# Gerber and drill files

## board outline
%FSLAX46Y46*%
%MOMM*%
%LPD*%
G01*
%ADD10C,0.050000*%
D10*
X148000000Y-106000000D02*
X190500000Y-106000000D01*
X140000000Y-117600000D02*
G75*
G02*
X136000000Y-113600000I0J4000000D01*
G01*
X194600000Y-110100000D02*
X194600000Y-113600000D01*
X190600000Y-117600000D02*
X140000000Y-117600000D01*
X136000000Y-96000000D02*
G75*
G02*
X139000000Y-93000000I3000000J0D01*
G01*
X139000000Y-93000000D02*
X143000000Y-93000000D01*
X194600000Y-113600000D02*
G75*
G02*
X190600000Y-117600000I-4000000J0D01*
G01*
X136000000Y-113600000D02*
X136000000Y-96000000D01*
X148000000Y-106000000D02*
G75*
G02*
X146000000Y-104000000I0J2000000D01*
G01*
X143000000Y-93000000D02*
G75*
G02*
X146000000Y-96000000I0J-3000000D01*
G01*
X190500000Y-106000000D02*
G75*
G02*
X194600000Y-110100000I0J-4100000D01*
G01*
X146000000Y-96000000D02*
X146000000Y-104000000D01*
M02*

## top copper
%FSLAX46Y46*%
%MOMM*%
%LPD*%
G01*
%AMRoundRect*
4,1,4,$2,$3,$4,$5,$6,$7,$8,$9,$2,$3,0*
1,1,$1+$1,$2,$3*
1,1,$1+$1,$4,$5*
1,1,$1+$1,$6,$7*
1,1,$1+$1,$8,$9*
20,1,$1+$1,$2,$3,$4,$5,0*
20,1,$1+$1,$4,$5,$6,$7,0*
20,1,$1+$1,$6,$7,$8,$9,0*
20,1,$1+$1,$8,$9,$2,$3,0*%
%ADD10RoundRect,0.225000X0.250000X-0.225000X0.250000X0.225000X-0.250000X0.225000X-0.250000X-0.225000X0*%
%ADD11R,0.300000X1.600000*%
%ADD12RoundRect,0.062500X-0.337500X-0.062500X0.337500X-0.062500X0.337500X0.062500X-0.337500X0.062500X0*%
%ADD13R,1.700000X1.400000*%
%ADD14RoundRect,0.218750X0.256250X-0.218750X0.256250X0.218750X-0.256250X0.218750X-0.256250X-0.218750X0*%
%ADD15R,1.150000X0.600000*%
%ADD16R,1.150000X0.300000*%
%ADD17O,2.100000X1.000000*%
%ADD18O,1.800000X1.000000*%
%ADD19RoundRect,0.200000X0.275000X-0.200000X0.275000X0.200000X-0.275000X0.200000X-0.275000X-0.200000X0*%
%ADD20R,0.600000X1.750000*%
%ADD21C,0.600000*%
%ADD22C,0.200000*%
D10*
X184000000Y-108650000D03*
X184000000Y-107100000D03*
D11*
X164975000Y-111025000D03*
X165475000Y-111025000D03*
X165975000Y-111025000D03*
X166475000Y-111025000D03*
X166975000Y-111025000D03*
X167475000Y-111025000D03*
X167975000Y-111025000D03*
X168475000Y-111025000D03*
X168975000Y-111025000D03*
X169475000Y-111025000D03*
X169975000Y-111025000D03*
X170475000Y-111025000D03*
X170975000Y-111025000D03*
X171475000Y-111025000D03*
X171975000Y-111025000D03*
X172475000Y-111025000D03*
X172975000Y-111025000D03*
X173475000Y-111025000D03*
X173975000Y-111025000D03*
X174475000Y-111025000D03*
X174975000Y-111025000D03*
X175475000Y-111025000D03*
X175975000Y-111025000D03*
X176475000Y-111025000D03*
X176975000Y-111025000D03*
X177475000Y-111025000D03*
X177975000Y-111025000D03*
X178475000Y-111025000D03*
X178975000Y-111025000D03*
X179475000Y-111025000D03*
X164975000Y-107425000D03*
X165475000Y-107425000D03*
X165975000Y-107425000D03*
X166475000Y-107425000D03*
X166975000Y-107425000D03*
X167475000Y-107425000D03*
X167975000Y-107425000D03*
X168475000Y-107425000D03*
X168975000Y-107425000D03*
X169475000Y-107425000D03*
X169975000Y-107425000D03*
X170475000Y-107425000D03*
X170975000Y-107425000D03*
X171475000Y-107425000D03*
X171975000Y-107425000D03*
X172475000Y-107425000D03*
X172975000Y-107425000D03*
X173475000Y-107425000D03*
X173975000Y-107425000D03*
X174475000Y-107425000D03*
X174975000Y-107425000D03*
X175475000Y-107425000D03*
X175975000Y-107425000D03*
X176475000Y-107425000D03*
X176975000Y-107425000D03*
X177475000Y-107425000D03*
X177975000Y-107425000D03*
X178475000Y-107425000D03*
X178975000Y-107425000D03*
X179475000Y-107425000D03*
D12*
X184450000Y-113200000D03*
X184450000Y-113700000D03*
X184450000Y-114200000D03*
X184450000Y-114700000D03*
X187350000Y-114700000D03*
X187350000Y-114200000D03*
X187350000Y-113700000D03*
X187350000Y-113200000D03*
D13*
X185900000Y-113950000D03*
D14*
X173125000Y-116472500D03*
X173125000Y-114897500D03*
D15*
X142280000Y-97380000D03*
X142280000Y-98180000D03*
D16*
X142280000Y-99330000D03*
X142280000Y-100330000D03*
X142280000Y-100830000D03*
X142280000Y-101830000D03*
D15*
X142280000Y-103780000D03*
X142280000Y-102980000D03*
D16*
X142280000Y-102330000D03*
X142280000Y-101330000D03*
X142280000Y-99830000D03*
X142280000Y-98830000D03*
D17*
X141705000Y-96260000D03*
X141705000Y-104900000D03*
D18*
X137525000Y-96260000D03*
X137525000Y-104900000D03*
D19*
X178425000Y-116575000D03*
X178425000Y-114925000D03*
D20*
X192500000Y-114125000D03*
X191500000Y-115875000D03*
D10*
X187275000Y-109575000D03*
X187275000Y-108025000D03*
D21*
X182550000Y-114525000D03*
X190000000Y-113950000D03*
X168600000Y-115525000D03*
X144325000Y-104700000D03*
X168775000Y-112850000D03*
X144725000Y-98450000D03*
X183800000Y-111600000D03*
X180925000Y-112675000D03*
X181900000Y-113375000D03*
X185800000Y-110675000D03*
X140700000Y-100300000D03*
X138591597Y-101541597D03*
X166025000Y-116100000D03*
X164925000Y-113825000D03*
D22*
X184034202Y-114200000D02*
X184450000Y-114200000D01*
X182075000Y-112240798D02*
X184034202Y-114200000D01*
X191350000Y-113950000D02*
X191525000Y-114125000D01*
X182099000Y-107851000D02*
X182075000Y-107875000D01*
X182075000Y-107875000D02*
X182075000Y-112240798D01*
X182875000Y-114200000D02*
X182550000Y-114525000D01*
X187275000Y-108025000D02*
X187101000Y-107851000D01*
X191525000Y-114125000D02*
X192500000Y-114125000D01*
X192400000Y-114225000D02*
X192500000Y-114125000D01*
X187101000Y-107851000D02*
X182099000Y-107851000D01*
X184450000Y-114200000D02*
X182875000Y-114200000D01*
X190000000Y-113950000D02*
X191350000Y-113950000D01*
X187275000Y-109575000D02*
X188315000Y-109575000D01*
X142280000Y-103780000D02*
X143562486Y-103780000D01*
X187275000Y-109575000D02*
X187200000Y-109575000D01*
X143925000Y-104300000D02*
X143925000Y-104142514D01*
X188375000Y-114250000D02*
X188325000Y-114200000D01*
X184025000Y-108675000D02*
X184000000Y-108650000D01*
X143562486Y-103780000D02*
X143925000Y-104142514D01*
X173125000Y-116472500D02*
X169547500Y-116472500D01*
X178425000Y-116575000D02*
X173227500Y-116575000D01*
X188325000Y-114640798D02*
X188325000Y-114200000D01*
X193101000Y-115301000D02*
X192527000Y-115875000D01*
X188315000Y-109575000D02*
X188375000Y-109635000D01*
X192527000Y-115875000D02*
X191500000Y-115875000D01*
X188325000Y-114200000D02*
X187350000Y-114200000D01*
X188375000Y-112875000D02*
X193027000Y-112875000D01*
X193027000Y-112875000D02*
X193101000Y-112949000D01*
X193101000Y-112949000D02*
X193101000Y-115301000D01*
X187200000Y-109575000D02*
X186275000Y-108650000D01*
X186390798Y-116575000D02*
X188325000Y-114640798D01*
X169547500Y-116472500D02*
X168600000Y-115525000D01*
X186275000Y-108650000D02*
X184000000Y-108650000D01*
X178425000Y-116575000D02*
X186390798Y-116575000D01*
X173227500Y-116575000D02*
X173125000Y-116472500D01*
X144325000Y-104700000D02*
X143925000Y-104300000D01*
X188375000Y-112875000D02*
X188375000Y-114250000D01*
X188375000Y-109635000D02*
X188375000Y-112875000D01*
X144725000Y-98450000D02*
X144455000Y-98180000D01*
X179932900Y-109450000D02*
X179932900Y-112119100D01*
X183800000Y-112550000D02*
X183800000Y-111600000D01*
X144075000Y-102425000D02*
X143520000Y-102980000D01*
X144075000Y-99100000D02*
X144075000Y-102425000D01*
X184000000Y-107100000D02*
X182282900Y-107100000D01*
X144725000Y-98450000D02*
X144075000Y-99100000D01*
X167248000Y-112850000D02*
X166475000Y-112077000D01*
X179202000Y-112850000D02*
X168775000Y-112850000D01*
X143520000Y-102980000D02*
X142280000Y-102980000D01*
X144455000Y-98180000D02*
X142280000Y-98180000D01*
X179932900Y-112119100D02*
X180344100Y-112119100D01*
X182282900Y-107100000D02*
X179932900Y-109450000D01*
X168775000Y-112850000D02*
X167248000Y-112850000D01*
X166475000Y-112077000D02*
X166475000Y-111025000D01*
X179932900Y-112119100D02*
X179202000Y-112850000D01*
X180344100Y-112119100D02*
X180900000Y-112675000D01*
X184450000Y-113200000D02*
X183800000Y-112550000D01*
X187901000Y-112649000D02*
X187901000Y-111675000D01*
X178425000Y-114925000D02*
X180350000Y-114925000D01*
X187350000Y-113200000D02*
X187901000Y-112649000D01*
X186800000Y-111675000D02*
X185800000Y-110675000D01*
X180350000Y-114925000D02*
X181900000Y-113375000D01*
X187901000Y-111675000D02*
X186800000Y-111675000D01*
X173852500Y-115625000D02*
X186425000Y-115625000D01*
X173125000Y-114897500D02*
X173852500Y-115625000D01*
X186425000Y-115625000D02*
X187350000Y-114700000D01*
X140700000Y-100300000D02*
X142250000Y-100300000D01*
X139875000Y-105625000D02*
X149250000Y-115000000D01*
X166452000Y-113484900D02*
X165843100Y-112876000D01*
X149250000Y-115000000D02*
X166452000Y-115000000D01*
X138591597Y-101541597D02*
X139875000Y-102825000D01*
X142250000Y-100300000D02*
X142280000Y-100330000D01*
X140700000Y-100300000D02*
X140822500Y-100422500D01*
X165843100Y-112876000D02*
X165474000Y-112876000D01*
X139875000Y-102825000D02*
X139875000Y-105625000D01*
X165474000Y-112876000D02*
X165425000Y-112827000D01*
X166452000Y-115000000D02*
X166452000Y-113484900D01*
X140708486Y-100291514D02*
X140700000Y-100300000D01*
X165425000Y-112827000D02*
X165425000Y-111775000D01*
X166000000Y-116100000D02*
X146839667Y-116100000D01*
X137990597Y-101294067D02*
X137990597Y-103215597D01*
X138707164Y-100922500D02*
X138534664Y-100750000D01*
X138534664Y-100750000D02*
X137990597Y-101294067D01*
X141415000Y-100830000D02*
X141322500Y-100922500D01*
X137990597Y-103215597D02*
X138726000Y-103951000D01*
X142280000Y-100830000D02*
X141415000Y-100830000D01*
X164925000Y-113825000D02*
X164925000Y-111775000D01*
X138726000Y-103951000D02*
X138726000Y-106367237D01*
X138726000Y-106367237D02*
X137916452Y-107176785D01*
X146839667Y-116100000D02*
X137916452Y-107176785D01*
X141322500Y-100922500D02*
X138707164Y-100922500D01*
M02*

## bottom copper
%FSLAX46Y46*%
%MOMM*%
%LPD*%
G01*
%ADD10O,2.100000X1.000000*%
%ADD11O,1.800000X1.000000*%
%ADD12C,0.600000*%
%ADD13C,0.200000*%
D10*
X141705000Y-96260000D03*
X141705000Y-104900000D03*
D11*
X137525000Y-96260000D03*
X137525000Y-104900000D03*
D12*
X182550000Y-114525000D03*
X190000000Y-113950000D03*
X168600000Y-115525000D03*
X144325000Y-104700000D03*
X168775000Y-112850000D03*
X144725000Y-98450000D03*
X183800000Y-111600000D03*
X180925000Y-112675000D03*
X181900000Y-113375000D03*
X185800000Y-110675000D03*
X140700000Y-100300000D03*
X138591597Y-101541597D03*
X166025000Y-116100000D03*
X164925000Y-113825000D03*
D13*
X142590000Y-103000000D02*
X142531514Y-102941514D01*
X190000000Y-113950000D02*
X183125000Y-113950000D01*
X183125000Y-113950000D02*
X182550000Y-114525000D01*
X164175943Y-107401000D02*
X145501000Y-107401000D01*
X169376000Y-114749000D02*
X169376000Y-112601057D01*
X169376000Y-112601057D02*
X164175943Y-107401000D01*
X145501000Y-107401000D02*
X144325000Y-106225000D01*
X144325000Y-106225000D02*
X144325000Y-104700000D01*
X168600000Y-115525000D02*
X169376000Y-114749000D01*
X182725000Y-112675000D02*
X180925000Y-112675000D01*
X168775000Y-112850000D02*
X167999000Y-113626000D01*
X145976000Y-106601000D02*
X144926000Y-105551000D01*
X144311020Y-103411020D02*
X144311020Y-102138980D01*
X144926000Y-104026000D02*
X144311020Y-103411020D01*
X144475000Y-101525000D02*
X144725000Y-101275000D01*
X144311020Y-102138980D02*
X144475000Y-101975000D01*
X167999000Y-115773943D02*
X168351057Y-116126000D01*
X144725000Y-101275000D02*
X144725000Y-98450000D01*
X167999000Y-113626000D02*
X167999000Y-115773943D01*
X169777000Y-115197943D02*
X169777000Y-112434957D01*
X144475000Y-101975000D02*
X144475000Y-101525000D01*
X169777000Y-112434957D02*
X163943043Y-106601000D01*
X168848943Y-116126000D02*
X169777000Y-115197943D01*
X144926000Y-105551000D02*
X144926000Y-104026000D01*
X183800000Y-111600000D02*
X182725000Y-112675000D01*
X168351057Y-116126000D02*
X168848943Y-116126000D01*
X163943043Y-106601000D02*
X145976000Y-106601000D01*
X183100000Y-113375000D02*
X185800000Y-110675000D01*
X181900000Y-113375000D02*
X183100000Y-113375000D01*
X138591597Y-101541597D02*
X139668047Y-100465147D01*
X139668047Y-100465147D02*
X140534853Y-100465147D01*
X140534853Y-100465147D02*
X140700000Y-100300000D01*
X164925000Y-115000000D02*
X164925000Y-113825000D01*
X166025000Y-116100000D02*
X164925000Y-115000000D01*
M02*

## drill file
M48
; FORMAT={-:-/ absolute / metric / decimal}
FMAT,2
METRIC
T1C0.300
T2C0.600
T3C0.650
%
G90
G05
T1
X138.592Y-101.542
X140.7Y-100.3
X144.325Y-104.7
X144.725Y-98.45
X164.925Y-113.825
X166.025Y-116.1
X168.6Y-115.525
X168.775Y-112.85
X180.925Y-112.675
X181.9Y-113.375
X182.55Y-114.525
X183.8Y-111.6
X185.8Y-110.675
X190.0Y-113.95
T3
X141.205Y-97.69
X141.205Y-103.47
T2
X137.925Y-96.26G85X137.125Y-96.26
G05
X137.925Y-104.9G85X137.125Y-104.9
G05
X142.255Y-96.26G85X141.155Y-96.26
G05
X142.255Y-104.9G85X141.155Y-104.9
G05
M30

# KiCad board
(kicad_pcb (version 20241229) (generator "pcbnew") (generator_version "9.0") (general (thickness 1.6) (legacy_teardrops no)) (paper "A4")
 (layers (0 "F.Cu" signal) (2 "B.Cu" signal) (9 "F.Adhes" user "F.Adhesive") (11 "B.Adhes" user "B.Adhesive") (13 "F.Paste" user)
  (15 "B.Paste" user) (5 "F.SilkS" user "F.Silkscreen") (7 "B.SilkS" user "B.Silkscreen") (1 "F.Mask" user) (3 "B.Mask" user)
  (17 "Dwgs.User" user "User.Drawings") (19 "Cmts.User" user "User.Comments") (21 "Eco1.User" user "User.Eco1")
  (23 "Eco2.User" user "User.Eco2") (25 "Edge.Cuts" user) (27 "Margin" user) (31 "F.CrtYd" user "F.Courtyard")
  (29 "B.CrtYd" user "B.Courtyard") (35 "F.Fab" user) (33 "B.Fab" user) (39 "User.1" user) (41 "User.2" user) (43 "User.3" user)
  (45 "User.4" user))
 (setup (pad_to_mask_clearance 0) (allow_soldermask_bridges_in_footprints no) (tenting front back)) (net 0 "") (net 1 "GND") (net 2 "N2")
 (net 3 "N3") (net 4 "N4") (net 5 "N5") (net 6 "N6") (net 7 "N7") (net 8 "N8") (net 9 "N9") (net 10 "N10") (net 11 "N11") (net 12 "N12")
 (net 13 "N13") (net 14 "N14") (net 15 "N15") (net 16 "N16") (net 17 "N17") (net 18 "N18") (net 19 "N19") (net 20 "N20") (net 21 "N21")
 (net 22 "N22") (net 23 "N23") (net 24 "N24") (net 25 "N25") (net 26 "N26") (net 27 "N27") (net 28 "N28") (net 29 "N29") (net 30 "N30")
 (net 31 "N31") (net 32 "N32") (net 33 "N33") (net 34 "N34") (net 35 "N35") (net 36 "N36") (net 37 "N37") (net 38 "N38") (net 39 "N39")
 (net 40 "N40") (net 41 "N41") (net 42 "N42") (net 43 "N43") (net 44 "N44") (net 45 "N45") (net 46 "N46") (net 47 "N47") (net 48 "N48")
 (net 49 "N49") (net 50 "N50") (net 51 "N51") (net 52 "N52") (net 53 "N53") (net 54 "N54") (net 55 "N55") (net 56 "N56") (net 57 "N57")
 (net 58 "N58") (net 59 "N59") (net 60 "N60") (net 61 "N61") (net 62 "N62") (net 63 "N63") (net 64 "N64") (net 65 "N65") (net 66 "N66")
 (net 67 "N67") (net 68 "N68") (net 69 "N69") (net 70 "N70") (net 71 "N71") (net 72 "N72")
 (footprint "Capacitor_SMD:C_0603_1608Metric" (layer "F.Cu") (at 184 107.875 90)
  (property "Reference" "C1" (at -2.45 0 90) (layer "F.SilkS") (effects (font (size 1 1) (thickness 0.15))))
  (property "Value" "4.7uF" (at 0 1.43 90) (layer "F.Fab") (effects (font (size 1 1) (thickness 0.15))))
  (pad "1" smd roundrect (at -0.775 0 90) (size 0.9 0.95) (layers "F.Cu" "F.Mask" "F.Paste") (roundrect_rratio 0.25) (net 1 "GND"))
  (pad "2" smd roundrect (at 0.775 0 90) (size 0.9 0.95) (layers "F.Cu" "F.Mask" "F.Paste") (roundrect_rratio 0.25) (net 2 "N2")))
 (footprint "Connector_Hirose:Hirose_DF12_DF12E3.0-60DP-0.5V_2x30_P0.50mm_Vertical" (layer "F.Cu") (at 172.225 109.225)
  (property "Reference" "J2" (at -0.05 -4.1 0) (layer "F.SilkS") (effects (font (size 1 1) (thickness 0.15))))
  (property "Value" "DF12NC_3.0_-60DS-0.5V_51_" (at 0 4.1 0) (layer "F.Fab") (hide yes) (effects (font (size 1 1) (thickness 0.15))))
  (pad "" smd rect (at -7.25 -2) (size 0.28 1.2) (layers "F.Paste"))
  (pad "" smd rect (at -7.25 2) (size 0.28 1.2) (layers "F.Paste"))
  (pad "" smd rect (at -6.75 -2) (size 0.28 1.2) (layers "F.Paste"))
  (pad "" smd rect (at -6.75 2) (size 0.28 1.2) (layers "F.Paste"))
  (pad "" smd rect (at -6.25 -2) (size 0.28 1.2) (layers "F.Paste"))
  (pad "" smd rect (at -6.25 2) (size 0.28 1.2) (layers "F.Paste"))
  (pad "" smd rect (at -5.75 -2) (size 0.28 1.2) (layers "F.Paste"))
  (pad "" smd rect (at -5.75 2) (size 0.28 1.2) (layers "F.Paste"))
  (pad "" smd rect (at -5.25 -2) (size 0.28 1.2) (layers "F.Paste"))
  (pad "" smd rect (at -5.25 2) (size 0.28 1.2) (layers "F.Paste"))
  (pad "" smd rect (at -4.75 -2) (size 0.28 1.2) (layers "F.Paste"))
  (pad "" smd rect (at -4.75 2) (size 0.28 1.2) (layers "F.Paste"))
  (pad "" smd rect (at -4.25 -2) (size 0.28 1.2) (layers "F.Paste"))
  (pad "" smd rect (at -4.25 2) (size 0.28 1.2) (layers "F.Paste"))
  (pad "" smd rect (at -3.75 -2) (size 0.28 1.2) (layers "F.Paste"))
  (pad "" smd rect (at -3.75 2) (size 0.28 1.2) (layers "F.Paste"))
  (pad "" smd rect (at -3.25 -2) (size 0.28 1.2) (layers "F.Paste"))
  (pad "" smd rect (at -3.25 2) (size 0.28 1.2) (layers "F.Paste"))
  (pad "" smd rect (at -2.75 -2) (size 0.28 1.2) (layers "F.Paste"))
  (pad "" smd rect (at -2.75 2) (size 0.28 1.2) (layers "F.Paste"))
  (pad "" smd rect (at -2.25 -2) (size 0.28 1.2) (layers "F.Paste"))
  (pad "" smd rect (at -2.25 2) (size 0.28 1.2) (layers "F.Paste"))
  (pad "" smd rect (at -1.75 -2) (size 0.28 1.2) (layers "F.Paste"))
  (pad "" smd rect (at -1.75 2) (size 0.28 1.2) (layers "F.Paste"))
  (pad "" smd rect (at -1.25 -2) (size 0.28 1.2) (layers "F.Paste"))
  (pad "" smd rect (at -1.25 2) (size 0.28 1.2) (layers "F.Paste"))
  (pad "" smd rect (at -0.75 -2) (size 0.28 1.2) (layers "F.Paste"))
  (pad "" smd rect (at -0.75 2) (size 0.28 1.2) (layers "F.Paste"))
  (pad "" smd rect (at -0.25 -2) (size 0.28 1.2) (layers "F.Paste"))
  (pad "" smd rect (at -0.25 2) (size 0.28 1.2) (layers "F.Paste"))
  (pad "" smd rect (at 0.25 -2) (size 0.28 1.2) (layers "F.Paste"))
  (pad "" smd rect (at 0.25 2) (size 0.28 1.2) (layers "F.Paste"))
  (pad "" smd rect (at 0.75 -2) (size 0.28 1.2) (layers "F.Paste"))
  (pad "" smd rect (at 0.75 2) (size 0.28 1.2) (layers "F.Paste"))
  (pad "" smd rect (at 1.25 -2) (size 0.28 1.2) (layers "F.Paste"))
  (pad "" smd rect (at 1.25 2) (size 0.28 1.2) (layers "F.Paste"))
  (pad "" smd rect (at 1.75 -2) (size 0.28 1.2) (layers "F.Paste"))
  (pad "" smd rect (at 1.75 2) (size 0.28 1.2) (layers "F.Paste"))
  (pad "" smd rect (at 2.25 -2) (size 0.28 1.2) (layers "F.Paste"))
  (pad "" smd rect (at 2.25 2) (size 0.28 1.2) (layers "F.Paste"))
  (pad "" smd rect (at 2.75 -2) (size 0.28 1.2) (layers "F.Paste"))
  (pad "" smd rect (at 2.75 2) (size 0.28 1.2) (layers "F.Paste"))
  (pad "" smd rect (at 3.25 -2) (size 0.28 1.2) (layers "F.Paste"))
  (pad "" smd rect (at 3.25 2) (size 0.28 1.2) (layers "F.Paste"))
  (pad "" smd rect (at 3.75 -2) (size 0.28 1.2) (layers "F.Paste"))
  (pad "" smd rect (at 3.75 2) (size 0.28 1.2) (layers "F.Paste"))
  (pad "" smd rect (at 4.25 -2) (size 0.28 1.2) (layers "F.Paste"))
  (pad "" smd rect (at 4.25 2) (size 0.28 1.2) (layers "F.Paste"))
  (pad "" smd rect (at 4.75 -2) (size 0.28 1.2) (layers "F.Paste"))
  (pad "" smd rect (at 4.75 2) (size 0.28 1.2) (layers "F.Paste"))
  (pad "" smd rect (at 5.25 -2) (size 0.28 1.2) (layers "F.Paste"))
  (pad "" smd rect (at 5.25 2) (size 0.28 1.2) (layers "F.Paste"))
  (pad "" smd rect (at 5.75 -2) (size 0.28 1.2) (layers "F.Paste"))
  (pad "" smd rect (at 5.75 2) (size 0.28 1.2) (layers "F.Paste"))
  (pad "" smd rect (at 6.25 -2) (size 0.28 1.2) (layers "F.Paste"))
  (pad "" smd rect (at 6.25 2) (size 0.28 1.2) (layers "F.Paste"))
  (pad "" smd rect (at 6.75 -2) (size 0.28 1.2) (layers "F.Paste"))
  (pad "" smd rect (at 6.75 2) (size 0.28 1.2) (layers "F.Paste"))
  (pad "" smd rect (at 7.25 -2) (size 0.28 1.2) (layers "F.Paste"))
  (pad "" smd rect (at 7.25 2) (size 0.28 1.2) (layers "F.Paste"))
  (pad "1" smd rect (at -7.25 1.8) (size 0.3 1.6) (layers "F.Cu" "F.Mask") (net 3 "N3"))
  (pad "2" smd rect (at -6.75 1.8) (size 0.3 1.6) (layers "F.Cu" "F.Mask") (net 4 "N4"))
  (pad "3" smd rect (at -6.25 1.8) (size 0.3 1.6) (layers "F.Cu" "F.Mask") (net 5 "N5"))
  (pad "4" smd rect (at -5.75 1.8) (size 0.3 1.6) (layers "F.Cu" "F.Mask") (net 2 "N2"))
  (pad "5" smd rect (at -5.25 1.8) (size 0.3 1.6) (layers "F.Cu" "F.Mask") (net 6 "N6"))
  (pad "6" smd rect (at -4.75 1.8) (size 0.3 1.6) (layers "F.Cu" "F.Mask") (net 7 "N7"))
  (pad "7" smd rect (at -4.25 1.8) (size 0.3 1.6) (layers "F.Cu" "F.Mask") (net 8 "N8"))
  (pad "8" smd rect (at -3.75 1.8) (size 0.3 1.6) (layers "F.Cu" "F.Mask") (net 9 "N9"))
  (pad "9" smd rect (at -3.25 1.8) (size 0.3 1.6) (layers "F.Cu" "F.Mask") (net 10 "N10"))
  (pad "10" smd rect (at -2.75 1.8) (size 0.3 1.6) (layers "F.Cu" "F.Mask") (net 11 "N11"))
  (pad "11" smd rect (at -2.25 1.8) (size 0.3 1.6) (layers "F.Cu" "F.Mask") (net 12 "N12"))
  (pad "12" smd rect (at -1.75 1.8) (size 0.3 1.6) (layers "F.Cu" "F.Mask") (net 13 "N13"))
  (pad "13" smd rect (at -1.25 1.8) (size 0.3 1.6) (layers "F.Cu" "F.Mask") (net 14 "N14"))
  (pad "14" smd rect (at -0.75 1.8) (size 0.3 1.6) (layers "F.Cu" "F.Mask") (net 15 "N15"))
  (pad "15" smd rect (at -0.25 1.8) (size 0.3 1.6) (layers "F.Cu" "F.Mask") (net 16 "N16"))
  (pad "16" smd rect (at 0.25 1.8) (size 0.3 1.6) (layers "F.Cu" "F.Mask") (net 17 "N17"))
  (pad "17" smd rect (at 0.75 1.8) (size 0.3 1.6) (layers "F.Cu" "F.Mask") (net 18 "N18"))
  (pad "18" smd rect (at 1.25 1.8) (size 0.3 1.6) (layers "F.Cu" "F.Mask") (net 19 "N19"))
  (pad "19" smd rect (at 1.75 1.8) (size 0.3 1.6) (layers "F.Cu" "F.Mask") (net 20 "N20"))
  (pad "20" smd rect (at 2.25 1.8) (size 0.3 1.6) (layers "F.Cu" "F.Mask") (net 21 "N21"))
  (pad "21" smd rect (at 2.75 1.8) (size 0.3 1.6) (layers "F.Cu" "F.Mask") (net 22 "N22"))
  (pad "22" smd rect (at 3.25 1.8) (size 0.3 1.6) (layers "F.Cu" "F.Mask") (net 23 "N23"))
  (pad "23" smd rect (at 3.75 1.8) (size 0.3 1.6) (layers "F.Cu" "F.Mask") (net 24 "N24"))
  (pad "24" smd rect (at 4.25 1.8) (size 0.3 1.6) (layers "F.Cu" "F.Mask") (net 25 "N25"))
  (pad "25" smd rect (at 4.75 1.8) (size 0.3 1.6) (layers "F.Cu" "F.Mask") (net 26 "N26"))
  (pad "26" smd rect (at 5.25 1.8) (size 0.3 1.6) (layers "F.Cu" "F.Mask") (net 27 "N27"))
  (pad "27" smd rect (at 5.75 1.8) (size 0.3 1.6) (layers "F.Cu" "F.Mask") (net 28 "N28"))
  (pad "28" smd rect (at 6.25 1.8) (size 0.3 1.6) (layers "F.Cu" "F.Mask") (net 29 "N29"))
  (pad "29" smd rect (at 6.75 1.8) (size 0.3 1.6) (layers "F.Cu" "F.Mask") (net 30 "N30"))
  (pad "30" smd rect (at 7.25 1.8) (size 0.3 1.6) (layers "F.Cu" "F.Mask") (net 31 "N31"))
  (pad "31" smd rect (at -7.25 -1.8) (size 0.3 1.6) (layers "F.Cu" "F.Mask") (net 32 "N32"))
  (pad "32" smd rect (at -6.75 -1.8) (size 0.3 1.6) (layers "F.Cu" "F.Mask") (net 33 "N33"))
  (pad "33" smd rect (at -6.25 -1.8) (size 0.3 1.6) (layers "F.Cu" "F.Mask") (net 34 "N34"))
  (pad "34" smd rect (at -5.75 -1.8) (size 0.3 1.6) (layers "F.Cu" "F.Mask") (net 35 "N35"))
  (pad "35" smd rect (at -5.25 -1.8) (size 0.3 1.6) (layers "F.Cu" "F.Mask") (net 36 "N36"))
  (pad "36" smd rect (at -4.75 -1.8) (size 0.3 1.6) (layers "F.Cu" "F.Mask") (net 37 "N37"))
  (pad "37" smd rect (at -4.25 -1.8) (size 0.3 1.6) (layers "F.Cu" "F.Mask") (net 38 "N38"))
  (pad "38" smd rect (at -3.75 -1.8) (size 0.3 1.6) (layers "F.Cu" "F.Mask") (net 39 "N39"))
  (pad "39" smd rect (at -3.25 -1.8) (size 0.3 1.6) (layers "F.Cu" "F.Mask") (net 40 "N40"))
  (pad "40" smd rect (at -2.75 -1.8) (size 0.3 1.6) (layers "F.Cu" "F.Mask") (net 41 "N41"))
  (pad "41" smd rect (at -2.25 -1.8) (size 0.3 1.6) (layers "F.Cu" "F.Mask") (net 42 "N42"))
  (pad "42" smd rect (at -1.75 -1.8) (size 0.3 1.6) (layers "F.Cu" "F.Mask") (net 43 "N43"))
  (pad "43" smd rect (at -1.25 -1.8) (size 0.3 1.6) (layers "F.Cu" "F.Mask") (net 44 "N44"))
  (pad "44" smd rect (at -0.75 -1.8) (size 0.3 1.6) (layers "F.Cu" "F.Mask") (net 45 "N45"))
  (pad "45" smd rect (at -0.25 -1.8) (size 0.3 1.6) (layers "F.Cu" "F.Mask") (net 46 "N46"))
  (pad "46" smd rect (at 0.25 -1.8) (size 0.3 1.6) (layers "F.Cu" "F.Mask") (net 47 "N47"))
  (pad "47" smd rect (at 0.75 -1.8) (size 0.3 1.6) (layers "F.Cu" "F.Mask") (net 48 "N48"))
  (pad "48" smd rect (at 1.25 -1.8) (size 0.3 1.6) (layers "F.Cu" "F.Mask") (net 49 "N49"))
  (pad "49" smd rect (at 1.75 -1.8) (size 0.3 1.6) (layers "F.Cu" "F.Mask") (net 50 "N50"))
  (pad "50" smd rect (at 2.25 -1.8) (size 0.3 1.6) (layers "F.Cu" "F.Mask") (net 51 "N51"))
  (pad "51" smd rect (at 2.75 -1.8) (size 0.3 1.6) (layers "F.Cu" "F.Mask") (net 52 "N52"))
  (pad "52" smd rect (at 3.25 -1.8) (size 0.3 1.6) (layers "F.Cu" "F.Mask") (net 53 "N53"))
  (pad "53" smd rect (at 3.75 -1.8) (size 0.3 1.6) (layers "F.Cu" "F.Mask") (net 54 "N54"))
  (pad "54" smd rect (at 4.25 -1.8) (size 0.3 1.6) (layers "F.Cu" "F.Mask") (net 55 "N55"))
  (pad "55" smd rect (at 4.75 -1.8) (size 0.3 1.6) (layers "F.Cu" "F.Mask") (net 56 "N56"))
  (pad "56" smd rect (at 5.25 -1.8) (size 0.3 1.6) (layers "F.Cu" "F.Mask") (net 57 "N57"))
  (pad "57" smd rect (at 5.75 -1.8) (size 0.3 1.6) (layers "F.Cu" "F.Mask") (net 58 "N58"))
  (pad "58" smd rect (at 6.25 -1.8) (size 0.3 1.6) (layers "F.Cu" "F.Mask") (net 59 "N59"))
  (pad "59" smd rect (at 6.75 -1.8) (size 0.3 1.6) (layers "F.Cu" "F.Mask") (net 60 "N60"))
  (pad "60" smd rect (at 7.25 -1.8) (size 0.3 1.6) (layers "F.Cu" "F.Mask") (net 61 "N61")))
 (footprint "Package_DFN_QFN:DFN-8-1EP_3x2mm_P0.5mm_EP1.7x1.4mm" (layer "F.Cu") (at 185.9 113.95)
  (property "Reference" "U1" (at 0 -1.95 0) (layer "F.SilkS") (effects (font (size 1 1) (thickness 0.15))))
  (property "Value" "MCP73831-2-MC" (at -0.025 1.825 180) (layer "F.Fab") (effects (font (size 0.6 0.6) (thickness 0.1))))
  (pad "" smd roundrect (at -0.425 -0.35) (size 0.69 0.56) (layers "F.Paste") (roundrect_rratio 0.25))
  (pad "" smd roundrect (at -0.425 0.35) (size 0.69 0.56) (layers "F.Paste") (roundrect_rratio 0.25))
  (pad "" smd roundrect (at 0.425 -0.35) (size 0.69 0.56) (layers "F.Paste") (roundrect_rratio 0.25))
  (pad "" smd roundrect (at 0.425 0.35) (size 0.69 0.56) (layers "F.Paste") (roundrect_rratio 0.25))
  (pad "1" smd roundrect (at -1.45 -0.75) (size 0.8 0.25) (layers "F.Cu" "F.Mask" "F.Paste") (roundrect_rratio 0.25) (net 2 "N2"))
  (pad "2" smd roundrect (at -1.45 -0.25) (size 0.8 0.25) (layers "F.Cu" "F.Mask" "F.Paste") (roundrect_rratio 0.25) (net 2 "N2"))
  (pad "3" smd roundrect (at -1.45 0.25) (size 0.8 0.25) (layers "F.Cu" "F.Mask" "F.Paste") (roundrect_rratio 0.25) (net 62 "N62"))
  (pad "4" smd roundrect (at -1.45 0.75) (size 0.8 0.25) (layers "F.Cu" "F.Mask" "F.Paste") (roundrect_rratio 0.25) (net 62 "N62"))
  (pad "5" smd roundrect (at 1.45 0.75) (size 0.8 0.25) (layers "F.Cu" "F.Mask" "F.Paste") (roundrect_rratio 0.25) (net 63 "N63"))
  (pad "6" smd roundrect (at 1.45 0.25) (size 0.8 0.25) (layers "F.Cu" "F.Mask" "F.Paste") (roundrect_rratio 0.25) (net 1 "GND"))
  (pad "7" smd roundrect (at 1.45 -0.25) (size 0.8 0.25) (layers "F.Cu" "F.Mask" "F.Paste") (roundrect_rratio 0.25) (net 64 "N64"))
  (pad "8" smd roundrect (at 1.45 -0.75) (size 0.8 0.25) (layers "F.Cu" "F.Mask" "F.Paste") (roundrect_rratio 0.25) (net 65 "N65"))
  (pad "9" smd rect (at 0 0) (size 1.7 1.4) (layers "F.Cu" "F.Mask") (zone_connect 2)))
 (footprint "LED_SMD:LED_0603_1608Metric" (layer "F.Cu") (at 173.125 115.685 90)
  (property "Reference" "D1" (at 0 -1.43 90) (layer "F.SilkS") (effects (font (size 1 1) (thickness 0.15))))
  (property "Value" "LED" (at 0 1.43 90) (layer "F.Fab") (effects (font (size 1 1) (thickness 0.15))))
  (pad "1" smd roundrect (at -0.7875 0 90) (size 0.875 0.95) (layers "F.Cu" "F.Mask" "F.Paste") (roundrect_rratio 0.25) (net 1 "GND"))
  (pad "2" smd roundrect (at 0.7875 0 90) (size 0.875 0.95) (layers "F.Cu" "F.Mask" "F.Paste") (roundrect_rratio 0.25) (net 63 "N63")))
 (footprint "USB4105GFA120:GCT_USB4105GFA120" (layer "F.Cu") (at 137.525 100.58 -90)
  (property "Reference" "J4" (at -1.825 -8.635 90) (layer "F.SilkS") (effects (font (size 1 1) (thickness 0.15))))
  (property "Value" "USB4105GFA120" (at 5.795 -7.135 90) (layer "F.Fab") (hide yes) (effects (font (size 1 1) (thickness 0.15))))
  (pad "" np_thru_hole circle (at -2.89 -3.68 270) (size 0.65 0.65) (drill 0.65) (layers "*.Cu" "*.Mask"))
  (pad "" np_thru_hole circle (at 2.89 -3.68 270) (size 0.65 0.65) (drill 0.65) (layers "*.Cu" "*.Mask"))
  (pad "A1_B12" smd rect (at -3.2 -4.755 270) (size 0.6 1.15) (layers "F.Cu" "F.Mask" "F.Paste") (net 1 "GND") (solder_mask_margin 0.102))
  (pad "A4_B9" smd rect (at -2.4 -4.755 270) (size 0.6 1.15) (layers "F.Cu" "F.Mask" "F.Paste") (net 2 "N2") (solder_mask_margin 0.102))
  (pad "A5" smd rect (at -1.25 -4.755 270) (size 0.3 1.15) (layers "F.Cu" "F.Mask" "F.Paste") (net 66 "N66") (solder_mask_margin 0.102))
  (pad "A6" smd rect (at -0.25 -4.755 270) (size 0.3 1.15) (layers "F.Cu" "F.Mask" "F.Paste") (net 4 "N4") (solder_mask_margin 0.102))
  (pad "A7" smd rect (at 0.25 -4.755 270) (size 0.3 1.15) (layers "F.Cu" "F.Mask" "F.Paste") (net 3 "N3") (solder_mask_margin 0.102))
  (pad "A8" smd rect (at 1.25 -4.755 270) (size 0.3 1.15) (layers "F.Cu" "F.Mask" "F.Paste") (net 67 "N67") (solder_mask_margin 0.102))
  (pad "B1_A12" smd rect (at 3.2 -4.755 270) (size 0.6 1.15) (layers "F.Cu" "F.Mask" "F.Paste") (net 1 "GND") (solder_mask_margin 0.102))
  (pad "B4_A9" smd rect (at 2.4 -4.755 270) (size 0.6 1.15) (layers "F.Cu" "F.Mask" "F.Paste") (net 2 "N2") (solder_mask_margin 0.102))
  (pad "B5" smd rect (at 1.75 -4.755 270) (size 0.3 1.15) (layers "F.Cu" "F.Mask" "F.Paste") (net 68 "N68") (solder_mask_margin 0.102))
  (pad "B6" smd rect (at 0.75 -4.755 270) (size 0.3 1.15) (layers "F.Cu" "F.Mask" "F.Paste") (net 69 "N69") (solder_mask_margin 0.102))
  (pad "B7" smd rect (at -0.75 -4.755 270) (size 0.3 1.15) (layers "F.Cu" "F.Mask" "F.Paste") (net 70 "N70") (solder_mask_margin 0.102))
  (pad "B8" smd rect (at -1.75 -4.755 270) (size 0.3 1.15) (layers "F.Cu" "F.Mask" "F.Paste") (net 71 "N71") (solder_mask_margin 0.102))
  (pad "SH1" thru_hole oval (at -4.32 -4.18 270) (size 1 2.1) (drill oval 0.6 1.7) (layers "*.Cu" "*.Mask") (remove_unused_layers no)
   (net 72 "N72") (solder_mask_margin 0.102))
  (pad "SH2" thru_hole oval (at 4.32 -4.18 270) (size 1 2.1) (drill oval 0.6 1.7) (layers "*.Cu" "*.Mask") (remove_unused_layers no)
   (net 72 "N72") (solder_mask_margin 0.102))
  (pad "SH3" thru_hole oval (at -4.32 0 270) (size 1 1.8) (drill oval 0.6 1.4) (layers "*.Cu" "*.Mask") (remove_unused_layers no)
   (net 72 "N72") (solder_mask_margin 0.102))
  (pad "SH4" thru_hole oval (at 4.32 0 270) (size 1 1.8) (drill oval 0.6 1.4) (layers "*.Cu" "*.Mask") (remove_unused_layers no)
   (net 72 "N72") (solder_mask_margin 0.102)))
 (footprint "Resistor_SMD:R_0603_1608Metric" (layer "F.Cu") (at 178.425 115.75 90)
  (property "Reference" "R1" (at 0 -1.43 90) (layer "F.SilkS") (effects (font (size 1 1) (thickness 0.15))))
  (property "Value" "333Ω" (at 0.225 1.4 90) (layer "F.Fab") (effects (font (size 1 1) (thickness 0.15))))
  (pad "1" smd roundrect (at -0.825 0 90) (size 0.8 0.95) (layers "F.Cu" "F.Mask" "F.Paste") (roundrect_rratio 0.25) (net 1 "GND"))
  (pad "2" smd roundrect (at 0.825 0 90) (size 0.8 0.95) (layers "F.Cu" "F.Mask" "F.Paste") (roundrect_rratio 0.25) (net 65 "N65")))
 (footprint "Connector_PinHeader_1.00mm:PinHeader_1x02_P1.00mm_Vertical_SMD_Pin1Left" (layer "F.Cu") (at 192 115 -90)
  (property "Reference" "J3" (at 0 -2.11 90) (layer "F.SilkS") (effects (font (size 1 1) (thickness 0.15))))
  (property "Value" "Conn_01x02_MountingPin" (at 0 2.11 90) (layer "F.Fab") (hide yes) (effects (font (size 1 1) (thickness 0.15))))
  (pad "1" smd rect (at -0.875 -0.5 270) (size 1.75 0.6) (layers "F.Cu" "F.Mask" "F.Paste") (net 62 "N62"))
  (pad "2" smd rect (at 0.875 0.5 270) (size 1.75 0.6) (layers "F.Cu" "F.Mask" "F.Paste") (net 1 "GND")))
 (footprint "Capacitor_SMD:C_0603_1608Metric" (layer "F.Cu") (at 187.275 108.8 90)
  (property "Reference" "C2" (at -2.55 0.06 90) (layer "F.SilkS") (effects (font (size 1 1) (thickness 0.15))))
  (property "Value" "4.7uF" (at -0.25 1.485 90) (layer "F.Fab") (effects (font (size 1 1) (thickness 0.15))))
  (pad "1" smd roundrect (at -0.775 0 90) (size 0.9 0.95) (layers "F.Cu" "F.Mask" "F.Paste") (roundrect_rratio 0.25) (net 1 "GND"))
  (pad "2" smd roundrect (at 0.775 0 90) (size 0.9 0.95) (layers "F.Cu" "F.Mask" "F.Paste") (roundrect_rratio 0.25) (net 62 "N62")))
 (gr_line (start 148 106) (end 190.5 106) (stroke (width 0.05) (type default)) (layer "Edge.Cuts"))
 (gr_arc (start 140 117.6) (mid 137.171573 116.428427) (end 136 113.6) (stroke (width 0.05) (type default)) (layer "Edge.Cuts"))
 (gr_line (start 194.6 110.1) (end 194.6 113.6) (stroke (width 0.05) (type solid)) (layer "Edge.Cuts"))
 (gr_line (start 190.6 117.6) (end 140 117.6) (stroke (width 0.05) (type default)) (layer "Edge.Cuts"))
 (gr_arc (start 136 96) (mid 136.87868 93.87868) (end 139 93) (stroke (width 0.05) (type default)) (layer "Edge.Cuts"))
 (gr_line (start 139 93) (end 143 93) (stroke (width 0.05) (type default)) (layer "Edge.Cuts"))
 (gr_arc (start 194.6 113.6) (mid 193.428427 116.428427) (end 190.6 117.6) (stroke (width 0.05) (type default)) (layer "Edge.Cuts"))
 (gr_line (start 136 113.6) (end 136 96) (stroke (width 0.05) (type default)) (layer "Edge.Cuts"))
 (gr_arc (start 148 106) (mid 146.585786 105.414214) (end 146 104) (stroke (width 0.05) (type default)) (layer "Edge.Cuts"))
 (gr_arc (start 143 93) (mid 145.12132 93.87868) (end 146 96) (stroke (width 0.05) (type default)) (layer "Edge.Cuts"))
 (gr_arc (start 190.5 106) (mid 193.399138 107.200862) (end 194.6 110.1) (stroke (width 0.05) (type default)) (layer "Edge.Cuts"))
 (gr_line (start 146 96) (end 146 104) (stroke (width 0.05) (type solid)) (layer "Edge.Cuts"))
 (segment (start 142.59 103) (end 142.531514 102.941514) (width 0.2) (layer "B.Cu") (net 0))
 (segment (start 184.034202 114.2) (end 184.45 114.2) (width 0.2) (layer "F.Cu") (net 62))
 (segment (start 182.075 112.240798) (end 184.034202 114.2) (width 0.2) (layer "F.Cu") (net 62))
 (segment (start 191.35 113.95) (end 191.525 114.125) (width 0.2) (layer "F.Cu") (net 62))
 (segment (start 182.099 107.851) (end 182.075 107.875) (width 0.2) (layer "F.Cu") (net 62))
 (segment (start 182.075 107.875) (end 182.075 112.240798) (width 0.2) (layer "F.Cu") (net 62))
 (segment (start 182.875 114.2) (end 182.55 114.525) (width 0.2) (layer "F.Cu") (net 62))
 (segment (start 187.275 108.025) (end 187.101 107.851) (width 0.2) (layer "F.Cu") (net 62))
 (segment (start 191.525 114.125) (end 192.5 114.125) (width 0.2) (layer "F.Cu") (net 62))
 (segment (start 192.4 114.225) (end 192.5 114.125) (width 0.2) (layer "F.Cu") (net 62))
 (segment (start 187.101 107.851) (end 182.099 107.851) (width 0.2) (layer "F.Cu") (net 62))
 (segment (start 184.45 114.2) (end 182.875 114.2) (width 0.2) (layer "F.Cu") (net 62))
 (segment (start 190 113.95) (end 191.35 113.95) (width 0.2) (layer "F.Cu") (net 62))
 (via (at 182.55 114.525) (size 0.6) (drill 0.3) (layers "F.Cu" "B.Cu") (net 62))
 (via (at 190 113.95) (size 0.6) (drill 0.3) (layers "F.Cu" "B.Cu") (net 62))
 (segment (start 190 113.95) (end 183.125 113.95) (width 0.2) (layer "B.Cu") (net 62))
 (segment (start 183.125 113.95) (end 182.55 114.525) (width 0.2) (layer "B.Cu") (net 62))
 (segment (start 187.275 109.575) (end 188.315 109.575) (width 0.2) (layer "F.Cu") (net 1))
 (segment (start 142.28 103.78) (end 143.562486 103.78) (width 0.2) (layer "F.Cu") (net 1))
 (segment (start 187.275 109.575) (end 187.2 109.575) (width 0.2) (layer "F.Cu") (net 1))
 (segment (start 143.925 104.3) (end 143.925 104.142514) (width 0.2) (layer "F.Cu") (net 1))
 (segment (start 188.375 114.25) (end 188.325 114.2) (width 0.2) (layer "F.Cu") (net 1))
 (segment (start 184.025 108.675) (end 184 108.65) (width 0.2) (layer "F.Cu") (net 1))
 (segment (start 143.562486 103.78) (end 143.925 104.142514) (width 0.2) (layer "F.Cu") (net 1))
 (segment (start 173.125 116.4725) (end 169.5475 116.4725) (width 0.2) (layer "F.Cu") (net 1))
 (segment (start 178.425 116.575) (end 173.2275 116.575) (width 0.2) (layer "F.Cu") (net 1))
 (segment (start 188.325 114.640798) (end 188.325 114.2) (width 0.2) (layer "F.Cu") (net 1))
 (segment (start 193.101 115.301) (end 192.527 115.875) (width 0.2) (layer "F.Cu") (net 1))
 (segment (start 188.315 109.575) (end 188.375 109.635) (width 0.2) (layer "F.Cu") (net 1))
 (segment (start 192.527 115.875) (end 191.5 115.875) (width 0.2) (layer "F.Cu") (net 1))
 (segment (start 188.325 114.2) (end 187.35 114.2) (width 0.2) (layer "F.Cu") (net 1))
 (segment (start 188.375 112.875) (end 193.027 112.875) (width 0.2) (layer "F.Cu") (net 1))
 (segment (start 193.027 112.875) (end 193.101 112.949) (width 0.2) (layer "F.Cu") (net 1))
 (segment (start 193.101 112.949) (end 193.101 115.301) (width 0.2) (layer "F.Cu") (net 1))
 (segment (start 187.2 109.575) (end 186.275 108.65) (width 0.2) (layer "F.Cu") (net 1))
 (segment (start 186.390798 116.575) (end 188.325 114.640798) (width 0.2) (layer "F.Cu") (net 1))
 (segment (start 169.5475 116.4725) (end 168.6 115.525) (width 0.2) (layer "F.Cu") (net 1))
 (segment (start 186.275 108.65) (end 184 108.65) (width 0.2) (layer "F.Cu") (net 1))
 (segment (start 178.425 116.575) (end 186.390798 116.575) (width 0.2) (layer "F.Cu") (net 1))
 (segment (start 173.2275 116.575) (end 173.125 116.4725) (width 0.2) (layer "F.Cu") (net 1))
 (segment (start 144.325 104.7) (end 143.925 104.3) (width 0.2) (layer "F.Cu") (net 1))
 (segment (start 188.375 112.875) (end 188.375 114.25) (width 0.2) (layer "F.Cu") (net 1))
 (segment (start 188.375 109.635) (end 188.375 112.875) (width 0.2) (layer "F.Cu") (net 1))
 (via (at 168.6 115.525) (size 0.6) (drill 0.3) (layers "F.Cu" "B.Cu") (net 1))
 (via (at 144.325 104.7) (size 0.6) (drill 0.3) (layers "F.Cu" "B.Cu") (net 1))
 (segment (start 164.175943 107.401) (end 145.501 107.401) (width 0.2) (layer "B.Cu") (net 1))
 (segment (start 169.376 114.749) (end 169.376 112.601057) (width 0.2) (layer "B.Cu") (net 1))
 (segment (start 169.376 112.601057) (end 164.175943 107.401) (width 0.2) (layer "B.Cu") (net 1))
 (segment (start 145.501 107.401) (end 144.325 106.225) (width 0.2) (layer "B.Cu") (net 1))
 (segment (start 144.325 106.225) (end 144.325 104.7) (width 0.2) (layer "B.Cu") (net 1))
 (segment (start 168.6 115.525) (end 169.376 114.749) (width 0.2) (layer "B.Cu") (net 1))
 (segment (start 144.725 98.45) (end 144.455 98.18) (width 0.2) (layer "F.Cu") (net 2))
 (segment (start 179.9329 109.45) (end 179.9329 112.1191) (width 0.2) (layer "F.Cu") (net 2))
 (segment (start 183.8 112.55) (end 183.8 111.6) (width 0.2) (layer "F.Cu") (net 2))
 (segment (start 144.075 102.425) (end 143.52 102.98) (width 0.2) (layer "F.Cu") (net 2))
 (segment (start 144.075 99.1) (end 144.075 102.425) (width 0.2) (layer "F.Cu") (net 2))
 (segment (start 184 107.1) (end 182.2829 107.1) (width 0.2) (layer "F.Cu") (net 2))
 (segment (start 144.725 98.45) (end 144.075 99.1) (width 0.2) (layer "F.Cu") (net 2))
 (segment (start 167.248 112.85) (end 166.475 112.077) (width 0.2) (layer "F.Cu") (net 2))
 (segment (start 179.202 112.85) (end 168.775 112.85) (width 0.2) (layer "F.Cu") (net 2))
 (segment (start 143.52 102.98) (end 142.28 102.98) (width 0.2) (layer "F.Cu") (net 2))
 (segment (start 144.455 98.18) (end 142.28 98.18) (width 0.2) (layer "F.Cu") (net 2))
 (segment (start 179.9329 112.1191) (end 180.3441 112.1191) (width 0.2) (layer "F.Cu") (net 2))
 (segment (start 182.2829 107.1) (end 179.9329 109.45) (width 0.2) (layer "F.Cu") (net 2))
 (segment (start 168.775 112.85) (end 167.248 112.85) (width 0.2) (layer "F.Cu") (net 2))
 (segment (start 166.475 112.077) (end 166.475 111.025) (width 0.2) (layer "F.Cu") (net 2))
 (segment (start 179.9329 112.1191) (end 179.202 112.85) (width 0.2) (layer "F.Cu") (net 2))
 (segment (start 180.3441 112.1191) (end 180.9 112.675) (width 0.2) (layer "F.Cu") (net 2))
 (segment (start 184.45 113.2) (end 183.8 112.55) (width 0.2) (layer "F.Cu") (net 2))
 (via (at 168.775 112.85) (size 0.6) (drill 0.3) (layers "F.Cu" "B.Cu") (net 2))
 (via (at 144.725 98.45) (size 0.6) (drill 0.3) (layers "F.Cu" "B.Cu") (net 2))
 (via (at 183.8 111.6) (size 0.6) (drill 0.3) (layers "F.Cu" "B.Cu") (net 2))
 (via (at 180.925 112.675) (size 0.6) (drill 0.3) (layers "F.Cu" "B.Cu") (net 2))
 (segment (start 182.725 112.675) (end 180.925 112.675) (width 0.2) (layer "B.Cu") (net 2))
 (segment (start 168.775 112.85) (end 167.999 113.626) (width 0.2) (layer "B.Cu") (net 2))
 (segment (start 145.976 106.601) (end 144.926 105.551) (width 0.2) (layer "B.Cu") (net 2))
 (segment (start 144.31102 103.41102) (end 144.31102 102.13898) (width 0.2) (layer "B.Cu") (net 2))
 (segment (start 144.926 104.026) (end 144.31102 103.41102) (width 0.2) (layer "B.Cu") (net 2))
 (segment (start 144.475 101.525) (end 144.725 101.275) (width 0.2) (layer "B.Cu") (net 2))
 (segment (start 144.31102 102.13898) (end 144.475 101.975) (width 0.2) (layer "B.Cu") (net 2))
 (segment (start 167.999 115.773943) (end 168.351057 116.126) (width 0.2) (layer "B.Cu") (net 2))
 (segment (start 144.725 101.275) (end 144.725 98.45) (width 0.2) (layer "B.Cu") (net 2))
 (segment (start 167.999 113.626) (end 167.999 115.773943) (width 0.2) (layer "B.Cu") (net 2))
 (segment (start 169.777 115.197943) (end 169.777 112.434957) (width 0.2) (layer "B.Cu") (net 2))
 (segment (start 144.475 101.975) (end 144.475 101.525) (width 0.2) (layer "B.Cu") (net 2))
 (segment (start 169.777 112.434957) (end 163.943043 106.601) (width 0.2) (layer "B.Cu") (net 2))
 (segment (start 168.848943 116.126) (end 169.777 115.197943) (width 0.2) (layer "B.Cu") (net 2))
 (segment (start 144.926 105.551) (end 144.926 104.026) (width 0.2) (layer "B.Cu") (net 2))
 (segment (start 183.8 111.6) (end 182.725 112.675) (width 0.2) (layer "B.Cu") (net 2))
 (segment (start 168.351057 116.126) (end 168.848943 116.126) (width 0.2) (layer "B.Cu") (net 2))
 (segment (start 163.943043 106.601) (end 145.976 106.601) (width 0.2) (layer "B.Cu") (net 2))
 (segment (start 187.901 112.649) (end 187.901 111.675) (width 0.2) (layer "F.Cu") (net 65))
 (segment (start 178.425 114.925) (end 180.35 114.925) (width 0.2) (layer "F.Cu") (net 65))
 (segment (start 187.35 113.2) (end 187.901 112.649) (width 0.2) (layer "F.Cu") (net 65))
 (segment (start 186.8 111.675) (end 185.8 110.675) (width 0.2) (layer "F.Cu") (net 65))
 (segment (start 180.35 114.925) (end 181.9 113.375) (width 0.2) (layer "F.Cu") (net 65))
 (segment (start 187.901 111.675) (end 186.8 111.675) (width 0.2) (layer "F.Cu") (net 65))
 (via (at 181.9 113.375) (size 0.6) (drill 0.3) (layers "F.Cu" "B.Cu") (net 65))
 (via (at 185.8 110.675) (size 0.6) (drill 0.3) (layers "F.Cu" "B.Cu") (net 65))
 (segment (start 183.1 113.375) (end 185.8 110.675) (width 0.2) (layer "B.Cu") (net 65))
 (segment (start 181.9 113.375) (end 183.1 113.375) (width 0.2) (layer "B.Cu") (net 65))
 (segment (start 173.8525 115.625) (end 186.425 115.625) (width 0.2) (layer "F.Cu") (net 63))
 (segment (start 173.125 114.8975) (end 173.8525 115.625) (width 0.2) (layer "F.Cu") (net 63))
 (segment (start 186.425 115.625) (end 187.35 114.7) (width 0.2) (layer "F.Cu") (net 63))
 (segment (start 140.7 100.3) (end 142.25 100.3) (width 0.2) (layer "F.Cu") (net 4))
 (segment (start 139.875 105.625) (end 149.25 115) (width 0.2) (layer "F.Cu") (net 4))
 (segment (start 166.452 113.4849) (end 165.8431 112.876) (width 0.2) (layer "F.Cu") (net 4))
 (segment (start 149.25 115) (end 166.452 115) (width 0.2) (layer "F.Cu") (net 4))
 (segment (start 138.591597 101.541597) (end 139.875 102.825) (width 0.2) (layer "F.Cu") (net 4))
 (segment (start 142.25 100.3) (end 142.28 100.33) (width 0.2) (layer "F.Cu") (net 4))
 (segment (start 140.7 100.3) (end 140.8225 100.4225) (width 0.2) (layer "F.Cu") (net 4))
 (segment (start 165.8431 112.876) (end 165.474 112.876) (width 0.2) (layer "F.Cu") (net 4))
 (segment (start 139.875 102.825) (end 139.875 105.625) (width 0.2) (layer "F.Cu") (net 4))
 (segment (start 165.474 112.876) (end 165.425 112.827) (width 0.2) (layer "F.Cu") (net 4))
 (segment (start 166.452 115) (end 166.452 113.4849) (width 0.2) (layer "F.Cu") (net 4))
 (segment (start 140.708486 100.291514) (end 140.7 100.3) (width 0.2) (layer "F.Cu") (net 4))
 (segment (start 165.425 112.827) (end 165.425 111.775) (width 0.2) (layer "F.Cu") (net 4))
 (via (at 140.7 100.3) (size 0.6) (drill 0.3) (layers "F.Cu" "B.Cu") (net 4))
 (via (at 138.591597 101.541597) (size 0.6) (drill 0.3) (layers "F.Cu" "B.Cu") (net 4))
 (segment (start 138.591597 101.541597) (end 139.668047 100.465147) (width 0.2) (layer "B.Cu") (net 4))
 (segment (start 139.668047 100.465147) (end 140.534853 100.465147) (width 0.2) (layer "B.Cu") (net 4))
 (segment (start 140.534853 100.465147) (end 140.7 100.3) (width 0.2) (layer "B.Cu") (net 4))
 (segment (start 166 116.1) (end 146.839667 116.1) (width 0.2) (layer "F.Cu") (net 3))
 (segment (start 137.990597 101.294067) (end 137.990597 103.215597) (width 0.2) (layer "F.Cu") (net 3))
 (segment (start 138.707164 100.9225) (end 138.534664 100.75) (width 0.2) (layer "F.Cu") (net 3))
 (segment (start 138.534664 100.75) (end 137.990597 101.294067) (width 0.2) (layer "F.Cu") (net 3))
 (segment (start 141.415 100.83) (end 141.3225 100.9225) (width 0.2) (layer "F.Cu") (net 3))
 (segment (start 137.990597 103.215597) (end 138.726 103.951) (width 0.2) (layer "F.Cu") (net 3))
 (segment (start 142.28 100.83) (end 141.415 100.83) (width 0.2) (layer "F.Cu") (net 3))
 (segment (start 164.925 113.825) (end 164.925 111.775) (width 0.2) (layer "F.Cu") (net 3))
 (segment (start 138.726 103.951) (end 138.726 106.367237) (width 0.2) (layer "F.Cu") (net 3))
 (segment (start 138.726 106.367237) (end 137.916452 107.176785) (width 0.2) (layer "F.Cu") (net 3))
 (segment (start 146.839667 116.1) (end 137.916452 107.176785) (width 0.2) (layer "F.Cu") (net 3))
 (segment (start 141.3225 100.9225) (end 138.707164 100.9225) (width 0.2) (layer "F.Cu") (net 3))
 (via (at 166.025 116.1) (size 0.6) (drill 0.3) (layers "F.Cu" "B.Cu") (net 3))
 (via (at 164.925 113.825) (size 0.6) (drill 0.3) (layers "F.Cu" "B.Cu") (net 3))
 (segment (start 164.925 115) (end 164.925 113.825) (width 0.2) (layer "B.Cu") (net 3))
 (segment (start 166.025 116.1) (end 164.925 115) (width 0.2) (layer "B.Cu") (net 3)))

